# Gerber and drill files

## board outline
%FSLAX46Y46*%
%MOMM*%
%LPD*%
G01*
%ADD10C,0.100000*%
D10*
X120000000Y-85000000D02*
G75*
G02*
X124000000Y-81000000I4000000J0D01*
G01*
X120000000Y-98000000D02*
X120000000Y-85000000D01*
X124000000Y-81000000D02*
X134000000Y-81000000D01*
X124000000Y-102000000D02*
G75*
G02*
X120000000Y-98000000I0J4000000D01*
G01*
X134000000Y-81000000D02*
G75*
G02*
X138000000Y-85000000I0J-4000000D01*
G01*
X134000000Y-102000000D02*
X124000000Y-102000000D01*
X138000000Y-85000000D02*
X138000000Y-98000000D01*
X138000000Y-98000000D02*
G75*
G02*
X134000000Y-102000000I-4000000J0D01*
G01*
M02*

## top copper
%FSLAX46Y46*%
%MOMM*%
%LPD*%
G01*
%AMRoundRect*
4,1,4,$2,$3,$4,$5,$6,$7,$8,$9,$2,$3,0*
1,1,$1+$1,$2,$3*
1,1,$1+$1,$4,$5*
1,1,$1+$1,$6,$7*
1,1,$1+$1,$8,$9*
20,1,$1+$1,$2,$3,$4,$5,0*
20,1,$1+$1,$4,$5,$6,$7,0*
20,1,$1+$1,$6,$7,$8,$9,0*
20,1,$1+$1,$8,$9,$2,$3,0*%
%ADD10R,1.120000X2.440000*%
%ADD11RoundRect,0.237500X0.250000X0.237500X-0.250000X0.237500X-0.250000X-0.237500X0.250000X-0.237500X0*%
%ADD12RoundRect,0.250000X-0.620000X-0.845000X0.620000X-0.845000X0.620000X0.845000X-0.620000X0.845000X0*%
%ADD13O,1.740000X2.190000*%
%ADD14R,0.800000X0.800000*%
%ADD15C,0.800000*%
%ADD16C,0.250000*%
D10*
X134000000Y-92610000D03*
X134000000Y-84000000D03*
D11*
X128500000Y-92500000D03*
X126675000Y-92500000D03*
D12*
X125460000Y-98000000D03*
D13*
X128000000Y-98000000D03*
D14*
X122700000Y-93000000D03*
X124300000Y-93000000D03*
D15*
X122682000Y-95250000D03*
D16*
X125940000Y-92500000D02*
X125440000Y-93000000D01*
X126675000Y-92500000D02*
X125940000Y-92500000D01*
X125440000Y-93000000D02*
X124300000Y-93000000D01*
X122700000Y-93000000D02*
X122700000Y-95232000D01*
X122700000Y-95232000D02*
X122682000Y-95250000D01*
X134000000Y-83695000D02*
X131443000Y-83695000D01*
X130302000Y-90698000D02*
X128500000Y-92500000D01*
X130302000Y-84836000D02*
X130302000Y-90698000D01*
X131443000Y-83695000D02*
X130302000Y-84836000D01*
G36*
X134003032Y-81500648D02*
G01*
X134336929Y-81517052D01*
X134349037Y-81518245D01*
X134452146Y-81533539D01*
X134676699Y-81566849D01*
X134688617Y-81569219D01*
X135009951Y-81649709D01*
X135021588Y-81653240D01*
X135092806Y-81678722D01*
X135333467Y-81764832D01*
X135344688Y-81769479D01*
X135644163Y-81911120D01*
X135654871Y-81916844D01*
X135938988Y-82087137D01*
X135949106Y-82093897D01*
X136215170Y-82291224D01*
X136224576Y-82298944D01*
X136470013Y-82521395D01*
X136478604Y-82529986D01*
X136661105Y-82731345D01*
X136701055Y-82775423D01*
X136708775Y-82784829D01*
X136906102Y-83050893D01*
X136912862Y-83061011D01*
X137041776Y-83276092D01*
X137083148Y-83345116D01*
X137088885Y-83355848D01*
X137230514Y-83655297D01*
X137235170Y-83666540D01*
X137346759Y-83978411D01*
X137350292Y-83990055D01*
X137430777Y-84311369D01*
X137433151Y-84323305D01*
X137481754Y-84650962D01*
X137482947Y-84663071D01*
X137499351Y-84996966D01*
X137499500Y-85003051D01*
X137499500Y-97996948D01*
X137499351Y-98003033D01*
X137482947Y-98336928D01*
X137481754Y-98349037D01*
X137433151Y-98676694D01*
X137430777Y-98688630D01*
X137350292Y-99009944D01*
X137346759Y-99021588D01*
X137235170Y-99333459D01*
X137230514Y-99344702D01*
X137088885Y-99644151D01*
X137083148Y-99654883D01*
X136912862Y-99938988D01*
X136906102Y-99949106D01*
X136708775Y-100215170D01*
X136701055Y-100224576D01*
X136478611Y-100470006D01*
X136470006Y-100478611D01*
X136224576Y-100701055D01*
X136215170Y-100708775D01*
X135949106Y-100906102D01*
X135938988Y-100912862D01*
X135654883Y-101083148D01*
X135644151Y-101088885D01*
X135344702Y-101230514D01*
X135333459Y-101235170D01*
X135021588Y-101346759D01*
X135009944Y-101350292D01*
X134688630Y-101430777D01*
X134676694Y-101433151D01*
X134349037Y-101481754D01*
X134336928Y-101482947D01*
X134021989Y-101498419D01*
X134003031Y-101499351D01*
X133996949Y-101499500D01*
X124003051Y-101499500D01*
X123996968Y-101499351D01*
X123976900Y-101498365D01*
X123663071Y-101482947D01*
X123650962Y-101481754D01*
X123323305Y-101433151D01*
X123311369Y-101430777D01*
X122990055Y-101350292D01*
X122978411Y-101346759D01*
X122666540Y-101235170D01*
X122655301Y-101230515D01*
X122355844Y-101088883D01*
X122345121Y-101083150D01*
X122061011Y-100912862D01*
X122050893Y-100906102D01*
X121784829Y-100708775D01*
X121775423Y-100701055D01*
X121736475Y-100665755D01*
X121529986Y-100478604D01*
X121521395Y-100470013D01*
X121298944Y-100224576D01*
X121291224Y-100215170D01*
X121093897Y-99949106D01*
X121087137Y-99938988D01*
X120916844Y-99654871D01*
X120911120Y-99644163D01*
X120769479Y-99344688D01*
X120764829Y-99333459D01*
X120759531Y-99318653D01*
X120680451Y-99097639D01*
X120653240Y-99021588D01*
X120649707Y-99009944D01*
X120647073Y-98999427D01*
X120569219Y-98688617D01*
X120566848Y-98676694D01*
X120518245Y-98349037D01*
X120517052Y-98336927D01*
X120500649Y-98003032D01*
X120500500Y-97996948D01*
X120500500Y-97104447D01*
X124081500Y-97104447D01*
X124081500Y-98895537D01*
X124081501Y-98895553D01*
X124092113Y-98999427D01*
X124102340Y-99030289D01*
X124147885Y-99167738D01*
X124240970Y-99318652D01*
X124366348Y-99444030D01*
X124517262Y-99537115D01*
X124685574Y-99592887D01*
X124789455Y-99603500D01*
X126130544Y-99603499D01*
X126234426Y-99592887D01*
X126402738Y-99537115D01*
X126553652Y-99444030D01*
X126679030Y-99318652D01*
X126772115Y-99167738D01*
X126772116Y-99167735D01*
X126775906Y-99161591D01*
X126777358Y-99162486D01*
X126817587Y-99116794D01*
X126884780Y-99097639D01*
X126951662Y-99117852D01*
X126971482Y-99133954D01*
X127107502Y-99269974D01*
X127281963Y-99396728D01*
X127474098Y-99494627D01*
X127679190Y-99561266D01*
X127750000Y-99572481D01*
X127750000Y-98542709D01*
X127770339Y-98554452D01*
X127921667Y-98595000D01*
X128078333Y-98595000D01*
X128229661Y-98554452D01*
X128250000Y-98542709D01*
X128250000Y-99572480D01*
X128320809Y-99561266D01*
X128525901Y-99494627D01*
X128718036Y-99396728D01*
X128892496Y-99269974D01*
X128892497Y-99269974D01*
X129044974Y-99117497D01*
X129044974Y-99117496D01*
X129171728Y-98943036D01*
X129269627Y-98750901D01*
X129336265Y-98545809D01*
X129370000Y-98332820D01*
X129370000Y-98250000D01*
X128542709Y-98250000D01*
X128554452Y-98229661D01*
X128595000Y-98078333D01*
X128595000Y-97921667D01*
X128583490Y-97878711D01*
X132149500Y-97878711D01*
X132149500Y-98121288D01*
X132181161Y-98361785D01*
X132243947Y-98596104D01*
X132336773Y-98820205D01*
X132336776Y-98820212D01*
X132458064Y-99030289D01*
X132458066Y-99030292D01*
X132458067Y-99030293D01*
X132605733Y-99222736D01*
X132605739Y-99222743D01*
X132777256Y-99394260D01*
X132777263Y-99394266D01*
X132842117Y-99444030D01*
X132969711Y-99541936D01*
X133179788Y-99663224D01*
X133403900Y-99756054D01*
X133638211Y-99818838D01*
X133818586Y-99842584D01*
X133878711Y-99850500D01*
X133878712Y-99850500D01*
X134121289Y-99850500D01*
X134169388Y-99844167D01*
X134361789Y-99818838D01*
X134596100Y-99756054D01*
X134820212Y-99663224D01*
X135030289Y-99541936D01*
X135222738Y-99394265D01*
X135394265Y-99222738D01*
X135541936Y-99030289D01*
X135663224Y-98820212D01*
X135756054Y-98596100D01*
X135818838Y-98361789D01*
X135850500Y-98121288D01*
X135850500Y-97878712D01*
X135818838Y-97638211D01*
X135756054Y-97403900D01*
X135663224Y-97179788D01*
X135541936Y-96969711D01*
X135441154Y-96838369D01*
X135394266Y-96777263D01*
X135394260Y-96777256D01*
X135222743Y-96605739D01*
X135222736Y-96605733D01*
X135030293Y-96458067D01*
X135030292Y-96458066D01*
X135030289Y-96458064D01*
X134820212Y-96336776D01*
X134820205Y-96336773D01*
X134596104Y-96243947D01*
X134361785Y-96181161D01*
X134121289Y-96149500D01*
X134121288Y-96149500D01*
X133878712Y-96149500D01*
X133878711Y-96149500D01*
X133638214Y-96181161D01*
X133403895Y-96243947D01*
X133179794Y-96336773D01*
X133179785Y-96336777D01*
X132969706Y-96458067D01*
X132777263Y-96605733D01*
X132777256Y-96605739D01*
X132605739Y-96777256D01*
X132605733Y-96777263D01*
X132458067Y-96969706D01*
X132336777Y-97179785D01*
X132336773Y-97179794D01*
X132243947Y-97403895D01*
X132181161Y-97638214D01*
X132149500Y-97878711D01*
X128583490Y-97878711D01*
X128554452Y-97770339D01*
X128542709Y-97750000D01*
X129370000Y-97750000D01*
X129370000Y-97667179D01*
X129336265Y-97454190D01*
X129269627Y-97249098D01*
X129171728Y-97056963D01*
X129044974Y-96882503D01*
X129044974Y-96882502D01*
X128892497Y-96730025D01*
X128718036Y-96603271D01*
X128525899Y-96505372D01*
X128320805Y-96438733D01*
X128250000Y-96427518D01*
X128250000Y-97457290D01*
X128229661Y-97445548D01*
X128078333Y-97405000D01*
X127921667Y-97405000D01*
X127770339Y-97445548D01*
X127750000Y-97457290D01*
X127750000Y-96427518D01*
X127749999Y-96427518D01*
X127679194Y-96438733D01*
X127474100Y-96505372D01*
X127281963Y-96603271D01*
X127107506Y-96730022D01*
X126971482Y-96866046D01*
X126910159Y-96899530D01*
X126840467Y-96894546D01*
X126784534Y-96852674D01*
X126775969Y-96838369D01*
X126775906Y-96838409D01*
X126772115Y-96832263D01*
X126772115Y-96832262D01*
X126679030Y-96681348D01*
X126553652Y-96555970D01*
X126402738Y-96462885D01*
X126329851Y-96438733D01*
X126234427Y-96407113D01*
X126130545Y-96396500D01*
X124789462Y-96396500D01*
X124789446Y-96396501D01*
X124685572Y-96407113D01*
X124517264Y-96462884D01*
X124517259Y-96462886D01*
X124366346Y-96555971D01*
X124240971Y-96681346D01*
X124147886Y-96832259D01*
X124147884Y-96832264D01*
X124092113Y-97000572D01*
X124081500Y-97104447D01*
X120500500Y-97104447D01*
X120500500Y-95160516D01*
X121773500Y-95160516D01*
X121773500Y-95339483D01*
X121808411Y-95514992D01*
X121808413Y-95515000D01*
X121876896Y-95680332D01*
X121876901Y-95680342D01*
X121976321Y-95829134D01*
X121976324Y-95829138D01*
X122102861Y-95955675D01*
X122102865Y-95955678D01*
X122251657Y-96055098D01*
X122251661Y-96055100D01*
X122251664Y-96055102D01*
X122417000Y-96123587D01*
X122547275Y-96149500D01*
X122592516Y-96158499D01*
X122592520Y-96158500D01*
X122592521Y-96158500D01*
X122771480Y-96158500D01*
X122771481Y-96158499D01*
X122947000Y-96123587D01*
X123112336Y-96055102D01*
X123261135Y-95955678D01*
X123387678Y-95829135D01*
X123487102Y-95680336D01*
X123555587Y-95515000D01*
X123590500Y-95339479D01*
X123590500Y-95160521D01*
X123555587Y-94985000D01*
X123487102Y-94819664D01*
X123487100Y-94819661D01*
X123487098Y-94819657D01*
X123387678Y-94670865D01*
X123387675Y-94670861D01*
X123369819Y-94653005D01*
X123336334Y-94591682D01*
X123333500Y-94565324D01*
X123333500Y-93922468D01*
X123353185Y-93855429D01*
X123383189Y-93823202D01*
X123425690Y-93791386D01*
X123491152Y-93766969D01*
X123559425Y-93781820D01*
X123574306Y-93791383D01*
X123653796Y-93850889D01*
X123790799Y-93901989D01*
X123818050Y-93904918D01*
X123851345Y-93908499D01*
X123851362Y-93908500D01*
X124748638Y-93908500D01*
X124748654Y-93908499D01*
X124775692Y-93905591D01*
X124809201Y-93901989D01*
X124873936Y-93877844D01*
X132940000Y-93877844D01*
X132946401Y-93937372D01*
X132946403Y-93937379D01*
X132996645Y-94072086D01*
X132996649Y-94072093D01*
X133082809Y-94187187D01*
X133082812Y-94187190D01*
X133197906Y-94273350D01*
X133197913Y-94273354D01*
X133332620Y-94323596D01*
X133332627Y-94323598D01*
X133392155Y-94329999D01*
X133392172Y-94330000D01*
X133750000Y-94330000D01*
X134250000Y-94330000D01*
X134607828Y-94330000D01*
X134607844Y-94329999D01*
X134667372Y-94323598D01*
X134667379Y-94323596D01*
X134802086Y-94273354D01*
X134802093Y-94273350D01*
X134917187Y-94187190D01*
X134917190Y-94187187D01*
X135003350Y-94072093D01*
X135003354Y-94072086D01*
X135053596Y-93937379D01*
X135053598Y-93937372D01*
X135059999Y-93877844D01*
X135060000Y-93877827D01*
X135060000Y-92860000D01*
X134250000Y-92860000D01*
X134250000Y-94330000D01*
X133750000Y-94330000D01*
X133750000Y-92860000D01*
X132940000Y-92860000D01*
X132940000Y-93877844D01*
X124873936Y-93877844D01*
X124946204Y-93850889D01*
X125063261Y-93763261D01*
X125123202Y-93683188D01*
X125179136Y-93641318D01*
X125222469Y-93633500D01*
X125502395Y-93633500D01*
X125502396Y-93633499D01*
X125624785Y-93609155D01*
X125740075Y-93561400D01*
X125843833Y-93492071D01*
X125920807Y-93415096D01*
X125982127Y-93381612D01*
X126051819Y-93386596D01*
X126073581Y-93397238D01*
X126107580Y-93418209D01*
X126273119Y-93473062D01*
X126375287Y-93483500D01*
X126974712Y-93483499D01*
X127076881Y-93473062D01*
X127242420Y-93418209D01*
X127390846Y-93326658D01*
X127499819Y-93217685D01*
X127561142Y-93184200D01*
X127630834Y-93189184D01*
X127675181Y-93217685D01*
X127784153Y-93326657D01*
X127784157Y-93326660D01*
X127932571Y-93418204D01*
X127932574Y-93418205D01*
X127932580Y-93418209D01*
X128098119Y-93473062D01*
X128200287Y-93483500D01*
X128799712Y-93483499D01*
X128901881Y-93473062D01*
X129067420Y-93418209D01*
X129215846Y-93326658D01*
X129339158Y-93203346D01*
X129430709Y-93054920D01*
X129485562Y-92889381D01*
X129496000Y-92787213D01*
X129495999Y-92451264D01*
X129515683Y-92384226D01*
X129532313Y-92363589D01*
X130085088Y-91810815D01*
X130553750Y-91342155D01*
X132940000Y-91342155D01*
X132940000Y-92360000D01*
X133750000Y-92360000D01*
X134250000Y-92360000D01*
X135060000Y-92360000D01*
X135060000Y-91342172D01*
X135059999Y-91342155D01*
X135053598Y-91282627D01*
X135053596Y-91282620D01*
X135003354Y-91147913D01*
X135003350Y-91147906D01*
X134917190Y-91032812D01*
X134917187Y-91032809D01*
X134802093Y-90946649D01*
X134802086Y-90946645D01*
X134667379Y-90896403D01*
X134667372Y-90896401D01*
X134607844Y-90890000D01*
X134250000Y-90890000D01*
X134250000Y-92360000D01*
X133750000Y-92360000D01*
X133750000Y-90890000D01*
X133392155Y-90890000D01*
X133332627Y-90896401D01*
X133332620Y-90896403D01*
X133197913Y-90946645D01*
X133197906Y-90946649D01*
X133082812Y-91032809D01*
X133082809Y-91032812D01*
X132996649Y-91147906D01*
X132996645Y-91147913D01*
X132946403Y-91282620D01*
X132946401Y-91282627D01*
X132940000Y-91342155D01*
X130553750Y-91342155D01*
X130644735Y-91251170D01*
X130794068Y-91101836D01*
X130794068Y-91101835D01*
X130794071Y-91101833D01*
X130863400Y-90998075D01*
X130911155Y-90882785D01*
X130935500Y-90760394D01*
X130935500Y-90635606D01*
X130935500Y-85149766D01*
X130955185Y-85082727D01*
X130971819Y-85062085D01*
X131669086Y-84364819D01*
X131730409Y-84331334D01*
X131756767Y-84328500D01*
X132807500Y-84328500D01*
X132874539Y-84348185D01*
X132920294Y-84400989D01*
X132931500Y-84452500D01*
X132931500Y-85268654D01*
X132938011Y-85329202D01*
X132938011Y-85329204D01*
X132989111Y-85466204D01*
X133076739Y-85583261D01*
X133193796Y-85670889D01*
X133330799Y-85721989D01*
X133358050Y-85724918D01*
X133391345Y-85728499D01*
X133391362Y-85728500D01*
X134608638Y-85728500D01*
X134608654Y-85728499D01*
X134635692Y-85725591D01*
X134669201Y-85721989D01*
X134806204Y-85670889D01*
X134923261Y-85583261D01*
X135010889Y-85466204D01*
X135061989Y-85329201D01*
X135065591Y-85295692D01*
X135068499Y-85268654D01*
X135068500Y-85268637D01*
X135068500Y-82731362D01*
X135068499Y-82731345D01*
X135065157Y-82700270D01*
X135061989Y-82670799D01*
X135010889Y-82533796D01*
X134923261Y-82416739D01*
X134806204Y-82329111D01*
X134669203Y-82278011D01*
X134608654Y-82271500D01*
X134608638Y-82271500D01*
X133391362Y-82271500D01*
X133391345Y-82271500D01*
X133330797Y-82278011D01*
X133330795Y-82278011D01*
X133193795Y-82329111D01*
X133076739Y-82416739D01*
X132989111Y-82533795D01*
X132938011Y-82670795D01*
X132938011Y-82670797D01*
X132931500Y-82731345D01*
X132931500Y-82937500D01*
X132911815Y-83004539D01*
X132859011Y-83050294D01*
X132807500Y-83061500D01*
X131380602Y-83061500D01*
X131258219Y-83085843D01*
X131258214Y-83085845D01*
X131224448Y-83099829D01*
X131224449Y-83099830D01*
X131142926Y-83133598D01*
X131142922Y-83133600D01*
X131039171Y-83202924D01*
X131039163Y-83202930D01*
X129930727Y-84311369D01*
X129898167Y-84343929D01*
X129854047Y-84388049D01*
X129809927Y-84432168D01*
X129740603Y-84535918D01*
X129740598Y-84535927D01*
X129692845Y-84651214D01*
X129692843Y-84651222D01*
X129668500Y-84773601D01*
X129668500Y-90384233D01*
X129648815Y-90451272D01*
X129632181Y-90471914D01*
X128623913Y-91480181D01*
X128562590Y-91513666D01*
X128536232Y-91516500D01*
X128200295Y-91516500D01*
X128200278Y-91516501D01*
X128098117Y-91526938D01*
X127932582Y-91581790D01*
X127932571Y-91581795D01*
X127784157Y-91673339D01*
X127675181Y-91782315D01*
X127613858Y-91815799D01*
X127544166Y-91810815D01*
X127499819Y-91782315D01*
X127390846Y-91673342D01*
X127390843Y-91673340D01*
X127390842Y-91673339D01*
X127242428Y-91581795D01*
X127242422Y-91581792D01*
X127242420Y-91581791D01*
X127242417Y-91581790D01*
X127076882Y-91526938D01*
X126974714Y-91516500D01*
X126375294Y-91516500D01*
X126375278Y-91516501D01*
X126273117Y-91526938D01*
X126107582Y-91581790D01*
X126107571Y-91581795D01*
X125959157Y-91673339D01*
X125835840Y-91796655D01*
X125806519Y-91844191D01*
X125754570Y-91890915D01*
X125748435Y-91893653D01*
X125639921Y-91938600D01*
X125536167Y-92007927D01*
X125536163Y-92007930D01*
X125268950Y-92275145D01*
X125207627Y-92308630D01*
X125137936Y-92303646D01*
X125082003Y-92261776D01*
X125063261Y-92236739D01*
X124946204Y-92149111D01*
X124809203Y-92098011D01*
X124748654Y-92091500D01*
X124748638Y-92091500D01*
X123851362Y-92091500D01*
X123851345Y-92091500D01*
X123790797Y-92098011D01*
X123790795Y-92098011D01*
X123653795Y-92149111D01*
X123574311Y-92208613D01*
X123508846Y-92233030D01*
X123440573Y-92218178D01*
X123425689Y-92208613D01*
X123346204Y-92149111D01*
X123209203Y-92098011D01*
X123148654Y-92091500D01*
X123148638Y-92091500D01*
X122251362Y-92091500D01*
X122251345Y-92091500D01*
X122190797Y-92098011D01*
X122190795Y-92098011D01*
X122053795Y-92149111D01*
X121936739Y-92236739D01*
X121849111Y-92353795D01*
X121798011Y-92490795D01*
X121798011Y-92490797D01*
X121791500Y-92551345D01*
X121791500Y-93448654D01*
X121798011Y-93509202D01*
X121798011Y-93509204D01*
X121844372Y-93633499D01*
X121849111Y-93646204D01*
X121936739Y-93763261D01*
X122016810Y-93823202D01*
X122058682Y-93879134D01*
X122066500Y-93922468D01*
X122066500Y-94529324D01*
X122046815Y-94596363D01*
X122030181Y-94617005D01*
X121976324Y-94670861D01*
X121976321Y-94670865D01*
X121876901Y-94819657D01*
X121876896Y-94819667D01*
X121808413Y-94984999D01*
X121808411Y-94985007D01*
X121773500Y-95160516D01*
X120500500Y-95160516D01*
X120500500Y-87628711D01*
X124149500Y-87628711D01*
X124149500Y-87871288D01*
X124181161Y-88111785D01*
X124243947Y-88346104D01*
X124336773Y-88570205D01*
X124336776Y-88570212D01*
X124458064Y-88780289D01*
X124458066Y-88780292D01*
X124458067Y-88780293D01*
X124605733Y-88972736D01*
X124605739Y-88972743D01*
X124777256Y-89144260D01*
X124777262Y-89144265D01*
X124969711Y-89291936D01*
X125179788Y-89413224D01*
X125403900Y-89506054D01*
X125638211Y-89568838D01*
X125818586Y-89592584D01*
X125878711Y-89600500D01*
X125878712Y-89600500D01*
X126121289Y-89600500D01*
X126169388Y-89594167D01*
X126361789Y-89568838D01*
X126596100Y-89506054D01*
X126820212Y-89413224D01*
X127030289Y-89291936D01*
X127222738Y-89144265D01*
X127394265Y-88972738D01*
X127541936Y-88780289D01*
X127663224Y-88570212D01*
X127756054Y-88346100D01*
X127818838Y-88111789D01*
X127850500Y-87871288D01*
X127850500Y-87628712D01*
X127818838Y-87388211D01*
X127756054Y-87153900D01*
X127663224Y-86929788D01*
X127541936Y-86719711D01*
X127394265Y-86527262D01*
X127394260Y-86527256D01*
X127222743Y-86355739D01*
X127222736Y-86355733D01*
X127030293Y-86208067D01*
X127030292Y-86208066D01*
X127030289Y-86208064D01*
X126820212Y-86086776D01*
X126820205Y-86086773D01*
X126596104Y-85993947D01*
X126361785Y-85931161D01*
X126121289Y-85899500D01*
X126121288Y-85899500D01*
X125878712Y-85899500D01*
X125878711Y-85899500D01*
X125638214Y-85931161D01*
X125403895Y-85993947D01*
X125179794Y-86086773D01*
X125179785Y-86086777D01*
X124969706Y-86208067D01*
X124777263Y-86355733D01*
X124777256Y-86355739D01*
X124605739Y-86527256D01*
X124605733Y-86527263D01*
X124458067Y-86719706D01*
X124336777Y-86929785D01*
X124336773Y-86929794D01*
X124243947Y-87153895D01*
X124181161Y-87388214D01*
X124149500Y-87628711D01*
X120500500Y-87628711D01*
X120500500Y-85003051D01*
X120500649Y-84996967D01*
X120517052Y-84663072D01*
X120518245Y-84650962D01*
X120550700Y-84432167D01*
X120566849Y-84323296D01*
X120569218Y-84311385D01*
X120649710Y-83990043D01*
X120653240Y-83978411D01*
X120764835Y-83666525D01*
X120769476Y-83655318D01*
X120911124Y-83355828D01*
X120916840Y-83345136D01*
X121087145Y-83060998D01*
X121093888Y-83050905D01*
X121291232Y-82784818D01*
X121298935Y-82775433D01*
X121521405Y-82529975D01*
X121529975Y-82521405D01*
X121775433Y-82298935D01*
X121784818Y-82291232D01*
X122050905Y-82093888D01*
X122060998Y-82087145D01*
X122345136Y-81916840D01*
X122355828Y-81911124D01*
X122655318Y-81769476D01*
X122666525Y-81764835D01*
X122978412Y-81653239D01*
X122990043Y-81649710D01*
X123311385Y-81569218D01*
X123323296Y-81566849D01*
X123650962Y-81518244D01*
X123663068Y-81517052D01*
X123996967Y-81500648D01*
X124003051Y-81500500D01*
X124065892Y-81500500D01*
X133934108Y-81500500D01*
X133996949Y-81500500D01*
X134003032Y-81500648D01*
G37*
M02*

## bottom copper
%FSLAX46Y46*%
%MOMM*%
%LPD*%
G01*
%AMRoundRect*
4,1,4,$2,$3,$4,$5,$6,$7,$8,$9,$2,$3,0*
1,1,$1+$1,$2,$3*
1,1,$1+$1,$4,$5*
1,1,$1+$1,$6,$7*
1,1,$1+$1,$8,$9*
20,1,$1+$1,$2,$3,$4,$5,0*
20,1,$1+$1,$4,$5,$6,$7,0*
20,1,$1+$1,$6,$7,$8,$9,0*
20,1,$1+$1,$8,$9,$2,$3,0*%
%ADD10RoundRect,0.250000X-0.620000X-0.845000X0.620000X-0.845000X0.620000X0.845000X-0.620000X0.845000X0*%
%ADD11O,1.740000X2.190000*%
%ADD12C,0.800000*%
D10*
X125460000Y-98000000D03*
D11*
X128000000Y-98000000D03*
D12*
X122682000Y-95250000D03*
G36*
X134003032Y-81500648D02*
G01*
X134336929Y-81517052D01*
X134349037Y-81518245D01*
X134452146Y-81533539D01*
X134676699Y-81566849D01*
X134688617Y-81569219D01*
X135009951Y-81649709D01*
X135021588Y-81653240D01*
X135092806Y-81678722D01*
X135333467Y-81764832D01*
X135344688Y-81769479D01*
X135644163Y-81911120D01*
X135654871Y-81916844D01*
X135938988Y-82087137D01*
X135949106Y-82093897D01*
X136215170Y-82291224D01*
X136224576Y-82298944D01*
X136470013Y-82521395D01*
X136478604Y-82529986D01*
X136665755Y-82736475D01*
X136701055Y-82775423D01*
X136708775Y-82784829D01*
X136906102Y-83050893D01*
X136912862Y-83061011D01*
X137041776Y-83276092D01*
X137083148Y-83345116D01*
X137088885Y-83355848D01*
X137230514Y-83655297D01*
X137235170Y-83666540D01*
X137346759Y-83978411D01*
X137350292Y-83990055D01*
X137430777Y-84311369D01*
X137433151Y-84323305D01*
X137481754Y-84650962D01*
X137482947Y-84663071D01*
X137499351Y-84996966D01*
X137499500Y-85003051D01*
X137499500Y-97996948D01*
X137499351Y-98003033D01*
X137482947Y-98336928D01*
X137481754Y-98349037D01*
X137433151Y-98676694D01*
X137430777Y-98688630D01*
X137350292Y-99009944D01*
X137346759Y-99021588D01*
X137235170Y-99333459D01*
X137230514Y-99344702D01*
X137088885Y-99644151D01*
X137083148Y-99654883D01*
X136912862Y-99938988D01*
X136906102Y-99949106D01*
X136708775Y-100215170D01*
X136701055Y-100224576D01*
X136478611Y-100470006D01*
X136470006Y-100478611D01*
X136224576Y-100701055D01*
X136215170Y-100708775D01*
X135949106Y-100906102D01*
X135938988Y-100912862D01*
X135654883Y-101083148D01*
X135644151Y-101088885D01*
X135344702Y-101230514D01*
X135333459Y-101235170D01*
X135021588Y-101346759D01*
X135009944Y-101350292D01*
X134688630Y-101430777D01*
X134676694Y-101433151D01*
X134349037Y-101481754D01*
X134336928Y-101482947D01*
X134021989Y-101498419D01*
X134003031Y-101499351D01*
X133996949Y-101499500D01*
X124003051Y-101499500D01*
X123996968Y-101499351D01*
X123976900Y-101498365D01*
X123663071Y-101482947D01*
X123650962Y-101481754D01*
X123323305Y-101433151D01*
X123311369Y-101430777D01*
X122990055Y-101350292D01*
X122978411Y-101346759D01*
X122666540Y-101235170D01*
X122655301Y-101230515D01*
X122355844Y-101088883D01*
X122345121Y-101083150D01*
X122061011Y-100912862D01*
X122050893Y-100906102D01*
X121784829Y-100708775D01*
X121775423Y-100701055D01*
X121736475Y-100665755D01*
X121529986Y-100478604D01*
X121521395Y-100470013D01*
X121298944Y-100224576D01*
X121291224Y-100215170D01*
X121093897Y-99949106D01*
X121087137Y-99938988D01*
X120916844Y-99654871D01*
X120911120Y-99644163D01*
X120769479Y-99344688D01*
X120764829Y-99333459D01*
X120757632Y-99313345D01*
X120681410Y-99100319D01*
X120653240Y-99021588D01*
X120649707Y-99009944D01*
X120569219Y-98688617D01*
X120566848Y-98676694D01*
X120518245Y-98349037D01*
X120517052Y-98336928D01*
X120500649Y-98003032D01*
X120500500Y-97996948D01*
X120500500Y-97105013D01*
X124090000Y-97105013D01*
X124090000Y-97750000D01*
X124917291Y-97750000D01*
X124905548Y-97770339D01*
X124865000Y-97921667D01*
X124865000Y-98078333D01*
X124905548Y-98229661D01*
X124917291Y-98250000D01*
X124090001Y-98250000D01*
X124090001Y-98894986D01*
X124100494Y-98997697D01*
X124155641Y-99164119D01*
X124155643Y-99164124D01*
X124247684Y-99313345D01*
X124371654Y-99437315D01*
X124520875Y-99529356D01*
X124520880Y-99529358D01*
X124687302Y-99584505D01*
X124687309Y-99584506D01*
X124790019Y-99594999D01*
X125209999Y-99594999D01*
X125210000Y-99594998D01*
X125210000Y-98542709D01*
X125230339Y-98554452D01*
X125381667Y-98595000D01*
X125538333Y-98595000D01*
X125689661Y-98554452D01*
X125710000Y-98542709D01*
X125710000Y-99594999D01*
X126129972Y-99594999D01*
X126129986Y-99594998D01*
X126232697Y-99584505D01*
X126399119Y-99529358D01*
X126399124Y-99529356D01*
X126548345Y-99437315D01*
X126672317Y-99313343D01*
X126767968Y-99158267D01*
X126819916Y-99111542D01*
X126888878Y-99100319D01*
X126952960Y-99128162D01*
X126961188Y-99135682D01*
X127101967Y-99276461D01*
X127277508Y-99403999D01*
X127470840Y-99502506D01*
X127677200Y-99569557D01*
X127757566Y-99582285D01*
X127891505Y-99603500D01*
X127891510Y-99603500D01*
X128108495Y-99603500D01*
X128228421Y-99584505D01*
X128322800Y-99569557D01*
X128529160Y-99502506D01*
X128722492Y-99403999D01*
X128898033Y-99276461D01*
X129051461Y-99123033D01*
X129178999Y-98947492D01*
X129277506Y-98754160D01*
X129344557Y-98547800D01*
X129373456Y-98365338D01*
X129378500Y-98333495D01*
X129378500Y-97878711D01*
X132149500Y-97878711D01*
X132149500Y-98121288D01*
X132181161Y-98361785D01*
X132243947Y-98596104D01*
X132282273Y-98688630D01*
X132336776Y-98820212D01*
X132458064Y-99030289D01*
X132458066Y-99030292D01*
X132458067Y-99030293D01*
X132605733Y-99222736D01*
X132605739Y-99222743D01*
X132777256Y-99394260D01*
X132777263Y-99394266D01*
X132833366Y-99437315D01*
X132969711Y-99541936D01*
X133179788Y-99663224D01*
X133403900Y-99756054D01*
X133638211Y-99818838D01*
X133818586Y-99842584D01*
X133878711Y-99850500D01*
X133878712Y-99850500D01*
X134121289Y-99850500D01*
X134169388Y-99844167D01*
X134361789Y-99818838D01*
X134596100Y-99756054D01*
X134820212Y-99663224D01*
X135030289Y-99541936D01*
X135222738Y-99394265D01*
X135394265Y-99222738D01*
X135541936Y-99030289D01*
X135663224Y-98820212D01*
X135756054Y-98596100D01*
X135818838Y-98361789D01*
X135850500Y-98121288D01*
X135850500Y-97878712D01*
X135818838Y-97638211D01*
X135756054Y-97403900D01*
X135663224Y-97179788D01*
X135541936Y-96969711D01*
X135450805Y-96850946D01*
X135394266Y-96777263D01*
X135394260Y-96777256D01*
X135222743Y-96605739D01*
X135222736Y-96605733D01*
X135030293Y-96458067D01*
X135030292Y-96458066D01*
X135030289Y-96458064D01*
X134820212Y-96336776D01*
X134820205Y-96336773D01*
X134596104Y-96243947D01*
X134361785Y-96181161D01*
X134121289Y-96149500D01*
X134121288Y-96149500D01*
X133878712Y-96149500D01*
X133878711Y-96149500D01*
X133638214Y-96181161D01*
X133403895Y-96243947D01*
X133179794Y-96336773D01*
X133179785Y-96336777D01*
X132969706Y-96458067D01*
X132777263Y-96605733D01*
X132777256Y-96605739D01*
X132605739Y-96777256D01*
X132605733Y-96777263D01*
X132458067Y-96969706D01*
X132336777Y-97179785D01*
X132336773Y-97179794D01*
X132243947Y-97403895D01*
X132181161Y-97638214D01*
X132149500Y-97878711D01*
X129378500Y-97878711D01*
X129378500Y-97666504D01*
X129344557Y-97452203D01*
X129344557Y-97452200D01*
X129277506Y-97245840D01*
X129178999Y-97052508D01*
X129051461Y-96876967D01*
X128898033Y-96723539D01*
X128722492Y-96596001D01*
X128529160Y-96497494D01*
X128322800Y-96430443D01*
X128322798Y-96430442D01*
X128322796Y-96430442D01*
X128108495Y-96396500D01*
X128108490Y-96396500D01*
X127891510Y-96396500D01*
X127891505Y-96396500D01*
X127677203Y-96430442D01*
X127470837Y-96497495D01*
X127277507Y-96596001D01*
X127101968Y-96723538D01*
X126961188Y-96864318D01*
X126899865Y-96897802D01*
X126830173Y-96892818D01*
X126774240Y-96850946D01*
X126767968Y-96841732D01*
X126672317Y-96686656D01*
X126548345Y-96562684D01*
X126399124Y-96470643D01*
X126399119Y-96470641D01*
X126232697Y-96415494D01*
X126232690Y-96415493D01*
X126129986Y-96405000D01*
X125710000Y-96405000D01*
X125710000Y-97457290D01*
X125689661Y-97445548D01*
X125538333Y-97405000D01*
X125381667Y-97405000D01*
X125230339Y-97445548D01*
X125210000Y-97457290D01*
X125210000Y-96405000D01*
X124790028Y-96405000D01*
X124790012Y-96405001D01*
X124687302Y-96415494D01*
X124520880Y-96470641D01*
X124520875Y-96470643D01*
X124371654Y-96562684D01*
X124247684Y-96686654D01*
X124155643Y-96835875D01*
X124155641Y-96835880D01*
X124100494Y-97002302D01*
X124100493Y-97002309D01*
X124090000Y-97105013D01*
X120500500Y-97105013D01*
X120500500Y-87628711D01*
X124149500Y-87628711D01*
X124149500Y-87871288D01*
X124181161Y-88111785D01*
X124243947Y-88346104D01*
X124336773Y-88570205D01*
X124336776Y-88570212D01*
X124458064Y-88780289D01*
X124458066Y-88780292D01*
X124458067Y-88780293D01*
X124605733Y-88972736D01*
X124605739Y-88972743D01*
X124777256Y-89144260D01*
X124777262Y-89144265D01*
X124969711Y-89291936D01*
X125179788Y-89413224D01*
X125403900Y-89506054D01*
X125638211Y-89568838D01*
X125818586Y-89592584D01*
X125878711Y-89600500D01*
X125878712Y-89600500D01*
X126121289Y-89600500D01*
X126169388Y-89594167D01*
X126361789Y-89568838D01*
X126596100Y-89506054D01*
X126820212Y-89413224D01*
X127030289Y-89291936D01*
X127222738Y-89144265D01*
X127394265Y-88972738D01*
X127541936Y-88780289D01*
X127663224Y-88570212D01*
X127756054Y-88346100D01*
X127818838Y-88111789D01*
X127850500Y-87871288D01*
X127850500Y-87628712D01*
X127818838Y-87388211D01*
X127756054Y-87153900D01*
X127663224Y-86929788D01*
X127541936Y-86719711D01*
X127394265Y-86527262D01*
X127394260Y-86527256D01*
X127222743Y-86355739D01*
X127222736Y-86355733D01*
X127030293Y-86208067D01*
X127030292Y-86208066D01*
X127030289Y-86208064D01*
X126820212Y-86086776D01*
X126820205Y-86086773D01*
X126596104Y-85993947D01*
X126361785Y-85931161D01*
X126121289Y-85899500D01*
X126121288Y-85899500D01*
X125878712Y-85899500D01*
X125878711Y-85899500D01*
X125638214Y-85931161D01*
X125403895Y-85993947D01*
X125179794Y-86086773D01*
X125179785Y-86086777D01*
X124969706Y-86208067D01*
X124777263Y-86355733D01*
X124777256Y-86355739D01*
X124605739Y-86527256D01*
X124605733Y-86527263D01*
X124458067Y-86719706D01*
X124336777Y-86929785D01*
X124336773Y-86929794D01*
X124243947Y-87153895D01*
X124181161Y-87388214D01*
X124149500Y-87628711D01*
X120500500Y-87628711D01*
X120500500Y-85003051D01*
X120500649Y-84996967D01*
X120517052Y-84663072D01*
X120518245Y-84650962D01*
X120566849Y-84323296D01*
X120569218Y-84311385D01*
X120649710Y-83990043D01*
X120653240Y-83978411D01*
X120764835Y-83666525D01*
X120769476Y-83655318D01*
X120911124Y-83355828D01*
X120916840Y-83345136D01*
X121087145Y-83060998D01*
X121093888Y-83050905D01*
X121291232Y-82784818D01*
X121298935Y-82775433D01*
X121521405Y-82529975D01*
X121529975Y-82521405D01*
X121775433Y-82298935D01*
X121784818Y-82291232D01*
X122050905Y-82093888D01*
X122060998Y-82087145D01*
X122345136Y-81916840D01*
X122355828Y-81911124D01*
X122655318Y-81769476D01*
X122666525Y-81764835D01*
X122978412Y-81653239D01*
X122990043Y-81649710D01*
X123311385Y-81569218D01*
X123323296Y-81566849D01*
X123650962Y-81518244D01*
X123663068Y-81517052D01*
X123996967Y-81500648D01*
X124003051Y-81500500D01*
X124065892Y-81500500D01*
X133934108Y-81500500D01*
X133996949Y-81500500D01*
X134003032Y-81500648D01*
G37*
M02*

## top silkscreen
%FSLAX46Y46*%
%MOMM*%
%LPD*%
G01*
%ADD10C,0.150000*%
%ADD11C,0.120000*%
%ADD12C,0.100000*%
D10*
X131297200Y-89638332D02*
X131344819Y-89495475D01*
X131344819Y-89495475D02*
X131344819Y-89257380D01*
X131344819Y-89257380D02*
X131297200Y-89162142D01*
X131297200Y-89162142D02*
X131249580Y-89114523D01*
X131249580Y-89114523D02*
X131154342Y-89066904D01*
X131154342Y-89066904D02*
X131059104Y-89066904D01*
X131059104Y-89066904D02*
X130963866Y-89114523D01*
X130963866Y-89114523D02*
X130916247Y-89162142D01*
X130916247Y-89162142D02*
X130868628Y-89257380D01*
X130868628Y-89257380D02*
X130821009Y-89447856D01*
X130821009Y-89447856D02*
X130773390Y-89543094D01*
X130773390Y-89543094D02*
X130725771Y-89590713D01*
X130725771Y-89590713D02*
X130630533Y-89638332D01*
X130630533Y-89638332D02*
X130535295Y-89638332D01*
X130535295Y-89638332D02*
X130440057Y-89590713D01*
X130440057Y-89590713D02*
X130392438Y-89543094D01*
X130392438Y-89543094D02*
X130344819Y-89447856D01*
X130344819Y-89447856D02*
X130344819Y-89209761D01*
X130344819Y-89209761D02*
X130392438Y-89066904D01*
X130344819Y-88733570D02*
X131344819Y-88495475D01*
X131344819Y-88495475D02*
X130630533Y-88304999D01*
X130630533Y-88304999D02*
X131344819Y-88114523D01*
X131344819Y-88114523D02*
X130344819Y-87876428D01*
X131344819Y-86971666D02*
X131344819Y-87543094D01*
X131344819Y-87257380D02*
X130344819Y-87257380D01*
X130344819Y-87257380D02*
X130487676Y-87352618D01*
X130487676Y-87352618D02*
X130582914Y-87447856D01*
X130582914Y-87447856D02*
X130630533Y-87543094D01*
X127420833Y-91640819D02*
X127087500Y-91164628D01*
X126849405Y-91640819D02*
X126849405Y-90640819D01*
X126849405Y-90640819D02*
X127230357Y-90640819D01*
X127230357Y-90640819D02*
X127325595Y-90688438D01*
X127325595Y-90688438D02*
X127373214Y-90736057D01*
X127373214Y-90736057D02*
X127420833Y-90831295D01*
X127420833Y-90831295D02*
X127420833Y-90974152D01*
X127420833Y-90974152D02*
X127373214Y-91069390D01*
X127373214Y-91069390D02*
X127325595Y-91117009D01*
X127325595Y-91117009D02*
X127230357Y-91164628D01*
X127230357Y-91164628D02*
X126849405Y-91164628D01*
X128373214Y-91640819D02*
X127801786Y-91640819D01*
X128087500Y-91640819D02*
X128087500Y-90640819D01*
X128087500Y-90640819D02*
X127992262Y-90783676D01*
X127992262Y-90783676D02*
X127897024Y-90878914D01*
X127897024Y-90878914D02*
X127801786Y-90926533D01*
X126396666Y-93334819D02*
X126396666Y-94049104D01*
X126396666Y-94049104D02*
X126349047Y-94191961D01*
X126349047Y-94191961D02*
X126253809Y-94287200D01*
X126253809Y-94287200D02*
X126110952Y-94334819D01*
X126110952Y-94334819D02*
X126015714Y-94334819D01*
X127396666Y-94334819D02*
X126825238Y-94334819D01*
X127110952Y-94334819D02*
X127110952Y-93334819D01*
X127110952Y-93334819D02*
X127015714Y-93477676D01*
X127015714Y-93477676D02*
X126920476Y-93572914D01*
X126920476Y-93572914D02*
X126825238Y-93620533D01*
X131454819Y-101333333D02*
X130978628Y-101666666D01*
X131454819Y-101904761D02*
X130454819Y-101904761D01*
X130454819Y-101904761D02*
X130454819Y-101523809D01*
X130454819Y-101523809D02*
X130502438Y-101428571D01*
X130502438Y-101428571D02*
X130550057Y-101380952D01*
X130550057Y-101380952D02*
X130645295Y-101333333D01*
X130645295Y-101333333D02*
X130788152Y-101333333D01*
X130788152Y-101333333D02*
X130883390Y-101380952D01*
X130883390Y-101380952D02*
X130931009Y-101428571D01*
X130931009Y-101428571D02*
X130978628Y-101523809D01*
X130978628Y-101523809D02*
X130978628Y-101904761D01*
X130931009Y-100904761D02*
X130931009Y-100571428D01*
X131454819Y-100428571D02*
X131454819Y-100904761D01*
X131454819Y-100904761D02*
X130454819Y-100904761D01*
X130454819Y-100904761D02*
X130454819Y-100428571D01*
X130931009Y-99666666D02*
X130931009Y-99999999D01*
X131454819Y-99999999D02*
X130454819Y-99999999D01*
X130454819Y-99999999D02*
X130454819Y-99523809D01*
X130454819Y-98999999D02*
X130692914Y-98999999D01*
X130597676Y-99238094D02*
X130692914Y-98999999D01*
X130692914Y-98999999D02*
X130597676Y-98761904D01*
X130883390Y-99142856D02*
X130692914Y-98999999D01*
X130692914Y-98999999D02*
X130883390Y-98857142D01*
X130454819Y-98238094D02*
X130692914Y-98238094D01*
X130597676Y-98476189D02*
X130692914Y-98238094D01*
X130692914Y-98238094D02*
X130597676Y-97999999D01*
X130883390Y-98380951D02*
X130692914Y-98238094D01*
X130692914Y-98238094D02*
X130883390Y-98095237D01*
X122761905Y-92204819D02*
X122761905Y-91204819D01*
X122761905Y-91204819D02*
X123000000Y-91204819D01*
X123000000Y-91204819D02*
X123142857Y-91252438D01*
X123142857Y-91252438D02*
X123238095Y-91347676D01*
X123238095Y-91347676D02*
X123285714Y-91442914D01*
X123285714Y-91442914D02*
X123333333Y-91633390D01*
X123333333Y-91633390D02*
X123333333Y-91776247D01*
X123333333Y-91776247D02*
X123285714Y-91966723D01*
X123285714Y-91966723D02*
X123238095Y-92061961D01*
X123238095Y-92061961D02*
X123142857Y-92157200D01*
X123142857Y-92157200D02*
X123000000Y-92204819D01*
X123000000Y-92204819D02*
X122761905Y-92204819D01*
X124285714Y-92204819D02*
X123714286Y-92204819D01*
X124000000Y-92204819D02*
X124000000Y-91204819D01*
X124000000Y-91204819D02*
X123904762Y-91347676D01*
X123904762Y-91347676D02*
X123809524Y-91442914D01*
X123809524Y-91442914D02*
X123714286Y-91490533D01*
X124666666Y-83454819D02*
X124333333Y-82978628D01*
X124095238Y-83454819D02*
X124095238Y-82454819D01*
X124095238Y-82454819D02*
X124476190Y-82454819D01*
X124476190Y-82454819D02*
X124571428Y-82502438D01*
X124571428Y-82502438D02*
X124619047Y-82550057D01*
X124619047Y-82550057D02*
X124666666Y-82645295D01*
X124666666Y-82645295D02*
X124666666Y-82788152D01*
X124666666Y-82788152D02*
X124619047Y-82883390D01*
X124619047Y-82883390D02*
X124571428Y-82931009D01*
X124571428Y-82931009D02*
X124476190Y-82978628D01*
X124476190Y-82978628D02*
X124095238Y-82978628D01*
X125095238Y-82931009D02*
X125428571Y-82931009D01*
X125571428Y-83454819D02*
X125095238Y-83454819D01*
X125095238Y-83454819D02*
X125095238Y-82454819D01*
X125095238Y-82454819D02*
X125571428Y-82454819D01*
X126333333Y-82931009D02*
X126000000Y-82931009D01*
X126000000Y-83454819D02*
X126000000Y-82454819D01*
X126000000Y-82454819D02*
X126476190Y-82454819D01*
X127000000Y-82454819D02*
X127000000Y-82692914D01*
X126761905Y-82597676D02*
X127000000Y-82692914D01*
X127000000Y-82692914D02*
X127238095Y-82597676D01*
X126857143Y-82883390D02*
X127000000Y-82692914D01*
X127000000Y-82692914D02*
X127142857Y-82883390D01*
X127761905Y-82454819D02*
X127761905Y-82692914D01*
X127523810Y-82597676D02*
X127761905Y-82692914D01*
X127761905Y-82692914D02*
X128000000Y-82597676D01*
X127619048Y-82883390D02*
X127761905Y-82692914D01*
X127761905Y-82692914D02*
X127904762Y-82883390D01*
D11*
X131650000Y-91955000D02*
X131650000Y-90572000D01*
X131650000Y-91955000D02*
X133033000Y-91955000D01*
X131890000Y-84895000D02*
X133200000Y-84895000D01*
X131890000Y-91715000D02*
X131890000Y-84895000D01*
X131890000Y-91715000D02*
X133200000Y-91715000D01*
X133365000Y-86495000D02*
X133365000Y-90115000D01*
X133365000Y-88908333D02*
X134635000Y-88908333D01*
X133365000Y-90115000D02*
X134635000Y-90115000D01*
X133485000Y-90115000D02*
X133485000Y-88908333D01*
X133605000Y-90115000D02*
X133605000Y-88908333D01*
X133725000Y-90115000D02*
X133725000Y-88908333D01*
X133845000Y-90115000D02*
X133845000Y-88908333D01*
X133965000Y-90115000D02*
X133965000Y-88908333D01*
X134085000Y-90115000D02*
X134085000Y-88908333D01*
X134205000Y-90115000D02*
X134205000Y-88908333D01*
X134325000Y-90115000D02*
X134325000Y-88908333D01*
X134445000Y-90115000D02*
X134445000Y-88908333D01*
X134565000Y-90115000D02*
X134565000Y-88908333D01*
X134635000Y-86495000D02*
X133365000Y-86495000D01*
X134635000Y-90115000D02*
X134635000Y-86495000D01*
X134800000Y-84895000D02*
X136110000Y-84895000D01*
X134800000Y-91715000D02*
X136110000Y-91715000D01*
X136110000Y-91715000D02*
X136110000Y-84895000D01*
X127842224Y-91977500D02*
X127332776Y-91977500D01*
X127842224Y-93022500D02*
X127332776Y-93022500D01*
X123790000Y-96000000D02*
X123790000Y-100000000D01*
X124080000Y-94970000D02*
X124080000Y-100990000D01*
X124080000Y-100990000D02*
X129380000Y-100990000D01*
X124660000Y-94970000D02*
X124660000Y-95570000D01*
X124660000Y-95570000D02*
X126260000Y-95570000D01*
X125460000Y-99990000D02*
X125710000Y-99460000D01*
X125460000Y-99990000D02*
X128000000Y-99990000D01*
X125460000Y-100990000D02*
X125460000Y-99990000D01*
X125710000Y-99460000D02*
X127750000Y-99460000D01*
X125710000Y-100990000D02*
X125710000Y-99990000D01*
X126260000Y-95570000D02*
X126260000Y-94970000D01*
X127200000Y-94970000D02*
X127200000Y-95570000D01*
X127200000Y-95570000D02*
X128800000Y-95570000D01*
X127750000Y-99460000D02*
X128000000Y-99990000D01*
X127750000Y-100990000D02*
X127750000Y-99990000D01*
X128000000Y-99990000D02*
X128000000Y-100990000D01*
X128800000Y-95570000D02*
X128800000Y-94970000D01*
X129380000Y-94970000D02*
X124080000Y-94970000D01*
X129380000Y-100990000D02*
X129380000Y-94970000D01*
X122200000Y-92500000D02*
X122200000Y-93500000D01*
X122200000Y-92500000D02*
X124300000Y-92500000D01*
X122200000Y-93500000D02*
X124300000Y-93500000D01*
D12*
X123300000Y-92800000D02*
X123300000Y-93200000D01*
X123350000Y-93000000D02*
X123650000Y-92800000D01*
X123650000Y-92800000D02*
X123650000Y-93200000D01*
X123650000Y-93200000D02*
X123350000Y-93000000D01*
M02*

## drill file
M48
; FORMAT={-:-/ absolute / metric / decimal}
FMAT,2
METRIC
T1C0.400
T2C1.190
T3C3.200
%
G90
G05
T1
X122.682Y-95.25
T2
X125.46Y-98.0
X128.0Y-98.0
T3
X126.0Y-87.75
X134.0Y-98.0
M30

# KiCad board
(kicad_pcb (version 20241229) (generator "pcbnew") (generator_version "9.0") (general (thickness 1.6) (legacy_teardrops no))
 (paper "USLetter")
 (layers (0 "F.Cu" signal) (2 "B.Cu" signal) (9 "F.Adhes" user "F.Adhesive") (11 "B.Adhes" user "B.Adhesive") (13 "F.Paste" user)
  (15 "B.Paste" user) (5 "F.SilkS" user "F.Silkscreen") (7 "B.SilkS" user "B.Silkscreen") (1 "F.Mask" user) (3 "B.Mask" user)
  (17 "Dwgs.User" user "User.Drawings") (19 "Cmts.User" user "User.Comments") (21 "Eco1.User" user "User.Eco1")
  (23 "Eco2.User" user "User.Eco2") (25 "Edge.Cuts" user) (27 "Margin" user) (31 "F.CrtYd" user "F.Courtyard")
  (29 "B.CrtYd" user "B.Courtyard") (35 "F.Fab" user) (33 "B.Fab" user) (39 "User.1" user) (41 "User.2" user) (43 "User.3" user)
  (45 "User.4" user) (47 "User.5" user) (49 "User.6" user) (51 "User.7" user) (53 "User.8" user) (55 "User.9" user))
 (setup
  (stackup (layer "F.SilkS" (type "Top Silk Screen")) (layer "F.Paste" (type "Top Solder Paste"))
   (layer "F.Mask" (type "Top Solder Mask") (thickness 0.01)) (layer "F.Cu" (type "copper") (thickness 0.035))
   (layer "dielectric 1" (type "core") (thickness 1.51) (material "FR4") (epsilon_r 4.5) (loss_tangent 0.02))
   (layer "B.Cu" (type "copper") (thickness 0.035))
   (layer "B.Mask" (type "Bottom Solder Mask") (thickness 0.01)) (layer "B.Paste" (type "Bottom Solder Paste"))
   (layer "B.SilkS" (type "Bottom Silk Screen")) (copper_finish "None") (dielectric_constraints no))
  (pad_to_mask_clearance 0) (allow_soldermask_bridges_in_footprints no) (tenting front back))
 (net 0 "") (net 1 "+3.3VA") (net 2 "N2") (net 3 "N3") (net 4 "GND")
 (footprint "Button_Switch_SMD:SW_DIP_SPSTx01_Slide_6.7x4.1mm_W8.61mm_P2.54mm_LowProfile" (layer "F.Cu") (at 134 88.305 90)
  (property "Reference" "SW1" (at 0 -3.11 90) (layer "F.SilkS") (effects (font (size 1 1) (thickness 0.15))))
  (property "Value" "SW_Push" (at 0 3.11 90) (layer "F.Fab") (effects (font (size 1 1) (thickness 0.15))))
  (fp_line (start -3.65 -2.35) (end -2.267 -2.35) (stroke (width 0.12) (type solid)) (layer "F.SilkS"))
  (fp_line (start -3.65 -2.35) (end -3.65 -0.967) (stroke (width 0.12) (type solid)) (layer "F.SilkS"))
  (fp_line (start 3.41 -2.11) (end 3.41 -0.8) (stroke (width 0.12) (type solid)) (layer "F.SilkS"))
  (fp_line (start -3.41 -2.11) (end 3.41 -2.11) (stroke (width 0.12) (type solid)) (layer "F.SilkS"))
  (fp_line (start -3.41 -2.11) (end -3.41 -0.8) (stroke (width 0.12) (type solid)) (layer "F.SilkS"))
  (fp_line (start 1.81 -0.635) (end -1.81 -0.635) (stroke (width 0.12) (type solid)) (layer "F.SilkS"))
  (fp_line (start -0.603333 -0.635) (end -0.603333 0.635) (stroke (width 0.12) (type solid)) (layer "F.SilkS"))
  (fp_line (start -1.81 -0.635) (end -1.81 0.635) (stroke (width 0.12) (type solid)) (layer "F.SilkS"))
  (fp_line (start -1.81 -0.515) (end -0.603333 -0.515) (stroke (width 0.12) (type solid)) (layer "F.SilkS"))
  (fp_line (start -1.81 -0.395) (end -0.603333 -0.395) (stroke (width 0.12) (type solid)) (layer "F.SilkS"))
  (fp_line (start -1.81 -0.275) (end -0.603333 -0.275) (stroke (width 0.12) (type solid)) (layer "F.SilkS"))
  (fp_line (start -1.81 -0.155) (end -0.603333 -0.155) (stroke (width 0.12) (type solid)) (layer "F.SilkS"))
  (fp_line (start -1.81 -0.035) (end -0.603333 -0.035) (stroke (width 0.12) (type solid)) (layer "F.SilkS"))
  (fp_line (start -1.81 0.085) (end -0.603333 0.085) (stroke (width 0.12) (type solid)) (layer "F.SilkS"))
  (fp_line (start -1.81 0.205) (end -0.603333 0.205) (stroke (width 0.12) (type solid)) (layer "F.SilkS"))
  (fp_line (start -1.81 0.325) (end -0.603333 0.325) (stroke (width 0.12) (type solid)) (layer "F.SilkS"))
  (fp_line (start -1.81 0.445) (end -0.603333 0.445) (stroke (width 0.12) (type solid)) (layer "F.SilkS"))
  (fp_line (start -1.81 0.565) (end -0.603333 0.565) (stroke (width 0.12) (type solid)) (layer "F.SilkS"))
  (fp_line (start 1.81 0.635) (end 1.81 -0.635) (stroke (width 0.12) (type solid)) (layer "F.SilkS"))
  (fp_line (start -1.81 0.635) (end 1.81 0.635) (stroke (width 0.12) (type solid)) (layer "F.SilkS"))
  (fp_line (start 3.41 0.8) (end 3.41 2.11) (stroke (width 0.12) (type solid)) (layer "F.SilkS"))
  (fp_line (start -3.41 0.8) (end -3.41 2.11) (stroke (width 0.12) (type solid)) (layer "F.SilkS"))
  (fp_line (start -3.41 2.11) (end 3.41 2.11) (stroke (width 0.12) (type solid)) (layer "F.SilkS"))
  (pad "1" smd rect (at -4.305 0 90) (size 2.44 1.12) (layers "F.Cu" "F.Mask" "F.Paste") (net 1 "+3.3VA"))
  (pad "2" smd rect (at 4.305 0 90) (size 2.44 1.12) (layers "F.Cu" "F.Mask" "F.Paste") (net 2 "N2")))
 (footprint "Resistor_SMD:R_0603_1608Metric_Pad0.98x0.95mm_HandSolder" (layer "F.Cu") (at 127.5875 92.5 180)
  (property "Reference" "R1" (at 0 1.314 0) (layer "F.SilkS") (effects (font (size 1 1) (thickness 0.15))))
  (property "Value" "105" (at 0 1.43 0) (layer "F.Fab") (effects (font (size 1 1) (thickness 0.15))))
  (fp_line (start -0.254724 0.5225) (end 0.254724 0.5225) (stroke (width 0.12) (type solid)) (layer "F.SilkS"))
  (fp_line (start -0.254724 -0.5225) (end 0.254724 -0.5225) (stroke (width 0.12) (type solid)) (layer "F.SilkS"))
  (pad "1" smd roundrect (at -0.9125 0 180) (size 0.975 0.95) (layers "F.Cu" "F.Mask" "F.Paste") (roundrect_rratio 0.25) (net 2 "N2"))
  (pad "2" smd roundrect (at 0.9125 0 180) (size 0.975 0.95) (layers "F.Cu" "F.Mask" "F.Paste") (roundrect_rratio 0.25) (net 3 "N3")))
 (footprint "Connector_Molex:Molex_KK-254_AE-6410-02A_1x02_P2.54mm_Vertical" (layer "F.Cu") (at 125.46 98)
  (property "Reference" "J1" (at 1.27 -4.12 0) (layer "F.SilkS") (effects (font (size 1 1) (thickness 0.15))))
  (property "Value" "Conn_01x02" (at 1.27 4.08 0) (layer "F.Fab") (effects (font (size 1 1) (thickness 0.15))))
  (fp_line (start -1.67 -2) (end -1.67 2) (stroke (width 0.12) (type solid)) (layer "F.SilkS"))
  (fp_line (start -1.38 -3.03) (end -1.38 2.99) (stroke (width 0.12) (type solid)) (layer "F.SilkS"))
  (fp_line (start -1.38 2.99) (end 3.92 2.99) (stroke (width 0.12) (type solid)) (layer "F.SilkS"))
  (fp_line (start -0.8 -3.03) (end -0.8 -2.43) (stroke (width 0.12) (type solid)) (layer "F.SilkS"))
  (fp_line (start -0.8 -2.43) (end 0.8 -2.43) (stroke (width 0.12) (type solid)) (layer "F.SilkS"))
  (fp_line (start 0 1.99) (end 0.25 1.46) (stroke (width 0.12) (type solid)) (layer "F.SilkS"))
  (fp_line (start 0 1.99) (end 2.54 1.99) (stroke (width 0.12) (type solid)) (layer "F.SilkS"))
  (fp_line (start 0 2.99) (end 0 1.99) (stroke (width 0.12) (type solid)) (layer "F.SilkS"))
  (fp_line (start 0.25 1.46) (end 2.29 1.46) (stroke (width 0.12) (type solid)) (layer "F.SilkS"))
  (fp_line (start 0.25 2.99) (end 0.25 1.99) (stroke (width 0.12) (type solid)) (layer "F.SilkS"))
  (fp_line (start 0.8 -2.43) (end 0.8 -3.03) (stroke (width 0.12) (type solid)) (layer "F.SilkS"))
  (fp_line (start 1.74 -3.03) (end 1.74 -2.43) (stroke (width 0.12) (type solid)) (layer "F.SilkS"))
  (fp_line (start 1.74 -2.43) (end 3.34 -2.43) (stroke (width 0.12) (type solid)) (layer "F.SilkS"))
  (fp_line (start 2.29 1.46) (end 2.54 1.99) (stroke (width 0.12) (type solid)) (layer "F.SilkS"))
  (fp_line (start 2.29 2.99) (end 2.29 1.99) (stroke (width 0.12) (type solid)) (layer "F.SilkS"))
  (fp_line (start 2.54 1.99) (end 2.54 2.99) (stroke (width 0.12) (type solid)) (layer "F.SilkS"))
  (fp_line (start 3.34 -2.43) (end 3.34 -3.03) (stroke (width 0.12) (type solid)) (layer "F.SilkS"))
  (fp_line (start 3.92 -3.03) (end -1.38 -3.03) (stroke (width 0.12) (type solid)) (layer "F.SilkS"))
  (fp_line (start 3.92 2.99) (end 3.92 -3.03) (stroke (width 0.12) (type solid)) (layer "F.SilkS"))
  (pad "1" thru_hole roundrect (at 0 0) (size 1.74 2.19) (drill 1.19) (layers "*.Cu" "*.Mask") (remove_unused_layers no)
   (roundrect_rratio 0.143678) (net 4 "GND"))
  (pad "2" thru_hole oval (at 2.54 0) (size 1.74 2.19) (drill 1.19) (layers "*.Cu" "*.Mask") (remove_unused_layers no) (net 1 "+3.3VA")))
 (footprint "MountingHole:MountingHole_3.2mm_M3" (layer "F.Cu") (at 134 98 90)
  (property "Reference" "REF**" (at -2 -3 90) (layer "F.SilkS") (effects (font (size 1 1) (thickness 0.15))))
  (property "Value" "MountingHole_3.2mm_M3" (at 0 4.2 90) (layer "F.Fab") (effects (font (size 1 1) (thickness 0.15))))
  (pad "" np_thru_hole circle (at 0 0 90) (size 3.2 3.2) (drill 3.2) (layers "*.Cu" "*.Mask")))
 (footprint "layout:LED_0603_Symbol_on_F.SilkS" (layer "F.Cu") (at 123.5 93)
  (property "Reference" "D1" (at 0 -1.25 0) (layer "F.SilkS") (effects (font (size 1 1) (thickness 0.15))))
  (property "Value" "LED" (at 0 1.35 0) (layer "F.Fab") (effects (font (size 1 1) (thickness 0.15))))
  (fp_line (start -1.3 -0.5) (end -1.3 0.5) (stroke (width 0.12) (type solid)) (layer "F.SilkS"))
  (fp_line (start -1.3 -0.5) (end 0.8 -0.5) (stroke (width 0.12) (type solid)) (layer "F.SilkS"))
  (fp_line (start -1.3 0.5) (end 0.8 0.5) (stroke (width 0.12) (type solid)) (layer "F.SilkS"))
  (fp_line (start -0.2 -0.2) (end -0.2 0.2) (stroke (width 0.1) (type solid)) (layer "F.SilkS"))
  (fp_line (start -0.15 0) (end 0.15 -0.2) (stroke (width 0.1) (type solid)) (layer "F.SilkS"))
  (fp_line (start 0.15 -0.2) (end 0.15 0.2) (stroke (width 0.1) (type solid)) (layer "F.SilkS"))
  (fp_line (start 0.15 0.2) (end -0.15 0) (stroke (width 0.1) (type solid)) (layer "F.SilkS"))
  (pad "1" smd rect (at -0.8 0 180) (size 0.8 0.8) (layers "F.Cu" "F.Mask" "F.Paste") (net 4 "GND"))
  (pad "2" smd rect (at 0.8 0 180) (size 0.8 0.8) (layers "F.Cu" "F.Mask" "F.Paste") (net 3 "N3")))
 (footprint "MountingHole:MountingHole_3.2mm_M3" (layer "F.Cu") (at 126 87.75)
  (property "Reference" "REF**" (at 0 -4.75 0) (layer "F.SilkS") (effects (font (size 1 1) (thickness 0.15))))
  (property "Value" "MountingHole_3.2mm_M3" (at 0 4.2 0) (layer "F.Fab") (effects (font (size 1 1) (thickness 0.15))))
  (pad "" np_thru_hole circle (at 0 0) (size 3.2 3.2) (drill 3.2) (layers "*.Cu" "*.Mask")))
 (gr_arc (start 120 85) (mid 121.171573 82.171573) (end 124 81) (stroke (width 0.1) (type default)) (layer "Edge.Cuts"))
 (gr_line (start 120 98) (end 120 85) (stroke (width 0.1) (type default)) (layer "Edge.Cuts"))
 (gr_line (start 124 81) (end 134 81) (stroke (width 0.1) (type default)) (layer "Edge.Cuts"))
 (gr_arc (start 124 102) (mid 121.171573 100.828427) (end 120 98) (stroke (width 0.1) (type default)) (layer "Edge.Cuts"))
 (gr_arc (start 134 81) (mid 136.828427 82.171573) (end 138 85) (stroke (width 0.1) (type default)) (layer "Edge.Cuts"))
 (gr_line (start 134 102) (end 124 102) (stroke (width 0.1) (type default)) (layer "Edge.Cuts"))
 (gr_line (start 138 85) (end 138 98) (stroke (width 0.1) (type default)) (layer "Edge.Cuts"))
 (gr_arc (start 138 98) (mid 136.828427 100.828427) (end 134 102) (stroke (width 0.1) (type default)) (layer "Edge.Cuts"))
 (segment (start 125.94 92.5) (end 125.44 93) (width 0.25) (layer "F.Cu") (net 3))
 (segment (start 126.675 92.5) (end 125.94 92.5) (width 0.25) (layer "F.Cu") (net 3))
 (segment (start 125.44 93) (end 124.3 93) (width 0.25) (layer "F.Cu") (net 3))
 (segment (start 122.7 93) (end 122.7 95.232) (width 0.25) (layer "F.Cu") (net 4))
 (segment (start 122.7 95.232) (end 122.682 95.25) (width 0.25) (layer "F.Cu") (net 4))
 (via (at 122.682 95.25) (size 0.8) (drill 0.4) (layers "F.Cu" "B.Cu") (free yes) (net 4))
 (segment (start 134 83.695) (end 131.443 83.695) (width 0.25) (layer "F.Cu") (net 2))
 (segment (start 130.302 90.698) (end 128.5 92.5) (width 0.25) (layer "F.Cu") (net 2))
 (segment (start 130.302 84.836) (end 130.302 90.698) (width 0.25) (layer "F.Cu") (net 2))
 (segment (start 131.443 83.695) (end 130.302 84.836) (width 0.25) (layer "F.Cu") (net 2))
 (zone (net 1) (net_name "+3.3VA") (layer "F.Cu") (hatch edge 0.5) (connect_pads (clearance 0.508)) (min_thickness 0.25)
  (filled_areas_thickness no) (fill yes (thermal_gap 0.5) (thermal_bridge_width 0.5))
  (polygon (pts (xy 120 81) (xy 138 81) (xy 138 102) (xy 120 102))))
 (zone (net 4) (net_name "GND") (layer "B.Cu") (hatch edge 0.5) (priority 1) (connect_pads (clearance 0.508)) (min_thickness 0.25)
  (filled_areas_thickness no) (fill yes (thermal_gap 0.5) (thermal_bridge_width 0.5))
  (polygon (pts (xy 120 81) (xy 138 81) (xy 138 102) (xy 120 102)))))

